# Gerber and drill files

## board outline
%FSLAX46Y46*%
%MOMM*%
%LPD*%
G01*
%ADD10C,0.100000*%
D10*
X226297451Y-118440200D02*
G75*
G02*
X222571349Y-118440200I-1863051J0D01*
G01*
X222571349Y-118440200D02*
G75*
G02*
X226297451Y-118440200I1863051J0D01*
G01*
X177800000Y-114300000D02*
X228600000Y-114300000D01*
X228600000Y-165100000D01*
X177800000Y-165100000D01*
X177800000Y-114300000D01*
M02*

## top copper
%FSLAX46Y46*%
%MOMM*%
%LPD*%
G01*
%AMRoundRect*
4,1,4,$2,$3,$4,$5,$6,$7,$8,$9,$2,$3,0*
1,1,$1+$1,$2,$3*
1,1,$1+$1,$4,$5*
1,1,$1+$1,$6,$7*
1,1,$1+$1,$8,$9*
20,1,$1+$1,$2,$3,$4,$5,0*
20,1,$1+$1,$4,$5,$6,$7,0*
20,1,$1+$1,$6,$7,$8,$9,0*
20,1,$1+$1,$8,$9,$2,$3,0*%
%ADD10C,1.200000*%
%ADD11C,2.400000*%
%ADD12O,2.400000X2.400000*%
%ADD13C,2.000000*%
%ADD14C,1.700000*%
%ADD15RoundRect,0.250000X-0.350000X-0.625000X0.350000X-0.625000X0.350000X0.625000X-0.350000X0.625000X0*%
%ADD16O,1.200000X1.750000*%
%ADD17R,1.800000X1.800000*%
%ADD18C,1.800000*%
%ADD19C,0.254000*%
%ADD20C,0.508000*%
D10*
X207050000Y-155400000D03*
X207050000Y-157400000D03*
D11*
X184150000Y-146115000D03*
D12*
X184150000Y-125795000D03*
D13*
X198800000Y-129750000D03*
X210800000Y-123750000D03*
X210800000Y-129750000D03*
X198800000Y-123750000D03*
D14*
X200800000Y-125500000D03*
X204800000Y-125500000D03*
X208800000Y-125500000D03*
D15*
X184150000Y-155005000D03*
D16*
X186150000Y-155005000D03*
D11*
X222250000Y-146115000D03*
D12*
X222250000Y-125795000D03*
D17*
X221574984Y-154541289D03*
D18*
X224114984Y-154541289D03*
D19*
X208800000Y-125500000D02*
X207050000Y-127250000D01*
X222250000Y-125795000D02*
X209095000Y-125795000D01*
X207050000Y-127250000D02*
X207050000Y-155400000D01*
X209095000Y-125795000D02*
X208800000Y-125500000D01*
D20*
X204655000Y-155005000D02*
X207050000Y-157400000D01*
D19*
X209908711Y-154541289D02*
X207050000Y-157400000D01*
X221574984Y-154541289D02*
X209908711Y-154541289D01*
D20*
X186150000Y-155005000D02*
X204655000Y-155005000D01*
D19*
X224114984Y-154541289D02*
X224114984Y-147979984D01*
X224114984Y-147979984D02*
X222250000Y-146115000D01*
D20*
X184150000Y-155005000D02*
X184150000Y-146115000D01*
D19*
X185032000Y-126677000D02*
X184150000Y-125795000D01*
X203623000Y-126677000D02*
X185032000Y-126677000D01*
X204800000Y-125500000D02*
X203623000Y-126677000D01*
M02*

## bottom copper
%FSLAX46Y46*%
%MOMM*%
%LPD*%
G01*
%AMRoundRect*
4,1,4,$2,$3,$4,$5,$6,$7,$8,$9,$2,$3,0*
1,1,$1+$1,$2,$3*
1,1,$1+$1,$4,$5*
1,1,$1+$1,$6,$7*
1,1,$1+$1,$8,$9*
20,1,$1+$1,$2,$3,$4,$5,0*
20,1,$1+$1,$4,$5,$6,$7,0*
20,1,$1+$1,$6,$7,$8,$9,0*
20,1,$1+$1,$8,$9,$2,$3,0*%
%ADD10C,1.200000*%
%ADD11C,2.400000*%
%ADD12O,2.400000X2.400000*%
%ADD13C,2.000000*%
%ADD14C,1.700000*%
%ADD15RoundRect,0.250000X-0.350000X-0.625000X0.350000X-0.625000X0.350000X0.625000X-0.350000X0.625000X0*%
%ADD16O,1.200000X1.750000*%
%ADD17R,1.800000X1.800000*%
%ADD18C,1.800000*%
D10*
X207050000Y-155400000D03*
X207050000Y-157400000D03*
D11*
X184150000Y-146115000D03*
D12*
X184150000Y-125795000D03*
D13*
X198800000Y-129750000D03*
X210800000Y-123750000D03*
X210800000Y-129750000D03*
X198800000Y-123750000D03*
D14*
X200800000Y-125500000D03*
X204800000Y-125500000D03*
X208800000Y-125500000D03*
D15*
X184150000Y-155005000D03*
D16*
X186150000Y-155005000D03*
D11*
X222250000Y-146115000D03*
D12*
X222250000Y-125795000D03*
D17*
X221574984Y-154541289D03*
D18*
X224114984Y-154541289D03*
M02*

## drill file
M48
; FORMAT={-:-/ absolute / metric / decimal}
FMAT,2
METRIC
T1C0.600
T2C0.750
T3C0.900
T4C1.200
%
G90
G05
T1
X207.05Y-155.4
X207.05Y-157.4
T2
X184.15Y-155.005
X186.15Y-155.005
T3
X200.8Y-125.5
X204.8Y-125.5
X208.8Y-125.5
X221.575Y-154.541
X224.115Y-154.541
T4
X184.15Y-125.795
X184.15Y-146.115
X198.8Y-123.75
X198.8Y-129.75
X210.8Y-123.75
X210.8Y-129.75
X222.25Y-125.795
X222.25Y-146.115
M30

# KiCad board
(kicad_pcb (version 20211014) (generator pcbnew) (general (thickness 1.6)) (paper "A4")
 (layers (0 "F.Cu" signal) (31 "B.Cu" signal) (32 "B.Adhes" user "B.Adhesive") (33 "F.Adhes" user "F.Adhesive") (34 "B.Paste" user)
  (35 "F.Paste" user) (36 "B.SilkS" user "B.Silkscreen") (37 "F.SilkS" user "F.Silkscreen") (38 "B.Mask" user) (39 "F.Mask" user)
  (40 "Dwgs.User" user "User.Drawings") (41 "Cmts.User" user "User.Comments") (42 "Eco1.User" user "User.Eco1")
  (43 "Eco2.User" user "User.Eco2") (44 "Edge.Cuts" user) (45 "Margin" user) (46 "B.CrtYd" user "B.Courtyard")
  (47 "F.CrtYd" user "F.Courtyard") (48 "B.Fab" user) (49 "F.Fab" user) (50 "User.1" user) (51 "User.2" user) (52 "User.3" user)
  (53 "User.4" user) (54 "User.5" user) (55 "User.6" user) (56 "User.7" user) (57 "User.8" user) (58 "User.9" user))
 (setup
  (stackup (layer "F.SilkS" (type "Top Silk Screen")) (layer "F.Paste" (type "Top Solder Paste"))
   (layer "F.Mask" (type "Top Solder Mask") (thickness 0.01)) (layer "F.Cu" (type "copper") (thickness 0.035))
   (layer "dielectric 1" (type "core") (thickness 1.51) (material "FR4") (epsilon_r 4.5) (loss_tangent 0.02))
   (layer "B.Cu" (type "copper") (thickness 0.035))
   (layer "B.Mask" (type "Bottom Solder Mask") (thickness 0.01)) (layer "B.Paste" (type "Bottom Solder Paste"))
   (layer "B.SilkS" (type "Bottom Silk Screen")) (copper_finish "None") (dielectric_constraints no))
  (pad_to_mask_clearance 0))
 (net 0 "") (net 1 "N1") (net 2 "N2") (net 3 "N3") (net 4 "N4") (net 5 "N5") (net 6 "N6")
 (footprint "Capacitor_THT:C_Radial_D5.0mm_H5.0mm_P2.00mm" (layer "F.Cu") (at 207.05 155.4 -90)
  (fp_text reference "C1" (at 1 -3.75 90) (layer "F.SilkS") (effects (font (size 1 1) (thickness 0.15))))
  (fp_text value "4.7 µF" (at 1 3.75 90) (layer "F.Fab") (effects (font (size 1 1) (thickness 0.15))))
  (pad "1" thru_hole circle (at 0 0 270) (size 1.2 1.2) (drill 0.6) (layers *.Cu *.Mask) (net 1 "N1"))
  (pad "2" thru_hole circle (at 2 0 270) (size 1.2 1.2) (drill 0.6) (layers *.Cu *.Mask) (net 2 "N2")))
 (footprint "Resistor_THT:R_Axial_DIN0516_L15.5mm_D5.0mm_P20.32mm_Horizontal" (layer "F.Cu") (at 184.15 146.115 90)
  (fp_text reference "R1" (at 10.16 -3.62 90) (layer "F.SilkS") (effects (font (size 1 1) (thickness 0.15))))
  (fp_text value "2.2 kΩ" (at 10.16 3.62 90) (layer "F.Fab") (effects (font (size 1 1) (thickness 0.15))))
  (pad "1" thru_hole circle (at 0 0 90) (size 2.4 2.4) (drill 1.2) (layers *.Cu *.Mask) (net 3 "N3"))
  (pad "2" thru_hole oval (at 20.32 0 90) (size 2.4 2.4) (drill 1.2) (layers *.Cu *.Mask) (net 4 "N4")))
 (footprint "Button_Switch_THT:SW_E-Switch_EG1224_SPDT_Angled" (layer "F.Cu") (at 200.8 125.5)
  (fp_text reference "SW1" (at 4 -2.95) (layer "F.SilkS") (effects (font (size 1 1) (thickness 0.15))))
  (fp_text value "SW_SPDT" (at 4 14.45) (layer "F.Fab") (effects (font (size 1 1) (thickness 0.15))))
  (pad "" thru_hole circle (at -2 4.25) (size 2 2) (drill 1.2) (layers *.Cu *.Mask))
  (pad "" thru_hole circle (at 10 -1.75) (size 2 2) (drill 1.2) (layers *.Cu *.Mask))
  (pad "" thru_hole circle (at 10 4.25) (size 2 2) (drill 1.2) (layers *.Cu *.Mask))
  (pad "" thru_hole circle (at -2 -1.75) (size 2 2) (drill 1.2) (layers *.Cu *.Mask))
  (pad "1" thru_hole circle (at 0 0) (size 1.7 1.7) (drill 0.9) (layers *.Cu *.Mask) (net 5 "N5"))
  (pad "2" thru_hole circle (at 4 0) (size 1.7 1.7) (drill 0.9) (layers *.Cu *.Mask) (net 4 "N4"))
  (pad "3" thru_hole circle (at 8 0) (size 1.7 1.7) (drill 0.9) (layers *.Cu *.Mask) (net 1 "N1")))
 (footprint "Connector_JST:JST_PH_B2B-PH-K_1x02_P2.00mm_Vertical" (layer "F.Cu") (at 184.15 155.005)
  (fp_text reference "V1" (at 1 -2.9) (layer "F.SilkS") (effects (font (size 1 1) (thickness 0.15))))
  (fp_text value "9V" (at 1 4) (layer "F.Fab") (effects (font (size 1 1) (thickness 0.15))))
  (pad "1" thru_hole roundrect (at 0 0) (size 1.2 1.75) (drill 0.75) (layers *.Cu *.Mask) (roundrect_rratio 0.208333) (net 3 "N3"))
  (pad "2" thru_hole oval (at 2 0) (size 1.2 1.75) (drill 0.75) (layers *.Cu *.Mask) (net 2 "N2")))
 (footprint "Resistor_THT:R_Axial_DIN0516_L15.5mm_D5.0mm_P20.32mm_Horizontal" (layer "F.Cu") (at 222.25 146.115 90)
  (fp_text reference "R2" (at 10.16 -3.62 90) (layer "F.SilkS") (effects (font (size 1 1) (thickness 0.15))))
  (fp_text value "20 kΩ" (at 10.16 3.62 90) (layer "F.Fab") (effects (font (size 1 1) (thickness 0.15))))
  (pad "1" thru_hole circle (at 0 0 90) (size 2.4 2.4) (drill 1.2) (layers *.Cu *.Mask) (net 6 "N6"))
  (pad "2" thru_hole oval (at 20.32 0 90) (size 2.4 2.4) (drill 1.2) (layers *.Cu *.Mask) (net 1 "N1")))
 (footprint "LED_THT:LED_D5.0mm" (layer "F.Cu") (at 221.574984 154.541289)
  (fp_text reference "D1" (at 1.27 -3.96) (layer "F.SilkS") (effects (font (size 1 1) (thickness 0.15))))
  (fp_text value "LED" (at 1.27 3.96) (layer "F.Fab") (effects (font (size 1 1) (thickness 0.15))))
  (pad "1" thru_hole rect (at 0 0) (size 1.8 1.8) (drill 0.9) (layers *.Cu *.Mask) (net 2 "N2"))
  (pad "2" thru_hole circle (at 2.54 0) (size 1.8 1.8) (drill 0.9) (layers *.Cu *.Mask) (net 6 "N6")))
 (gr_circle (center 224.4344 118.4402) (end 226.1108 119.253) (layer "Edge.Cuts") (width 0.1) (fill none))
 (gr_rect (start 177.8 114.3) (end 228.6 165.1) (layer "Edge.Cuts") (width 0.1) (fill none))
 (segment (start 208.8 125.5) (end 207.05 127.25) (width 0.254) (layer "F.Cu") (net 1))
 (segment (start 222.25 125.795) (end 209.095 125.795) (width 0.254) (layer "F.Cu") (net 1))
 (segment (start 207.05 127.25) (end 207.05 155.4) (width 0.254) (layer "F.Cu") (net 1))
 (segment (start 209.095 125.795) (end 208.8 125.5) (width 0.254) (layer "F.Cu") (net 1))
 (segment (start 204.655 155.005) (end 207.05 157.4) (width 0.508) (layer "F.Cu") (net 2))
 (segment (start 209.908711 154.541289) (end 207.05 157.4) (width 0.254) (layer "F.Cu") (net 2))
 (segment (start 221.574984 154.541289) (end 209.908711 154.541289) (width 0.254) (layer "F.Cu") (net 2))
 (segment (start 186.15 155.005) (end 204.655 155.005) (width 0.508) (layer "F.Cu") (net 2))
 (segment (start 224.114984 154.541289) (end 224.114984 147.979984) (width 0.254) (layer "F.Cu") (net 6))
 (segment (start 224.114984 147.979984) (end 222.25 146.115) (width 0.254) (layer "F.Cu") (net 6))
 (segment (start 184.15 155.005) (end 184.15 146.115) (width 0.508) (layer "F.Cu") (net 3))
 (segment (start 185.032 126.677) (end 184.15 125.795) (width 0.254) (layer "F.Cu") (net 4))
 (segment (start 203.623 126.677) (end 185.032 126.677) (width 0.254) (layer "F.Cu") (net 4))
 (segment (start 204.8 125.5) (end 203.623 126.677) (width 0.254) (layer "F.Cu") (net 4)))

